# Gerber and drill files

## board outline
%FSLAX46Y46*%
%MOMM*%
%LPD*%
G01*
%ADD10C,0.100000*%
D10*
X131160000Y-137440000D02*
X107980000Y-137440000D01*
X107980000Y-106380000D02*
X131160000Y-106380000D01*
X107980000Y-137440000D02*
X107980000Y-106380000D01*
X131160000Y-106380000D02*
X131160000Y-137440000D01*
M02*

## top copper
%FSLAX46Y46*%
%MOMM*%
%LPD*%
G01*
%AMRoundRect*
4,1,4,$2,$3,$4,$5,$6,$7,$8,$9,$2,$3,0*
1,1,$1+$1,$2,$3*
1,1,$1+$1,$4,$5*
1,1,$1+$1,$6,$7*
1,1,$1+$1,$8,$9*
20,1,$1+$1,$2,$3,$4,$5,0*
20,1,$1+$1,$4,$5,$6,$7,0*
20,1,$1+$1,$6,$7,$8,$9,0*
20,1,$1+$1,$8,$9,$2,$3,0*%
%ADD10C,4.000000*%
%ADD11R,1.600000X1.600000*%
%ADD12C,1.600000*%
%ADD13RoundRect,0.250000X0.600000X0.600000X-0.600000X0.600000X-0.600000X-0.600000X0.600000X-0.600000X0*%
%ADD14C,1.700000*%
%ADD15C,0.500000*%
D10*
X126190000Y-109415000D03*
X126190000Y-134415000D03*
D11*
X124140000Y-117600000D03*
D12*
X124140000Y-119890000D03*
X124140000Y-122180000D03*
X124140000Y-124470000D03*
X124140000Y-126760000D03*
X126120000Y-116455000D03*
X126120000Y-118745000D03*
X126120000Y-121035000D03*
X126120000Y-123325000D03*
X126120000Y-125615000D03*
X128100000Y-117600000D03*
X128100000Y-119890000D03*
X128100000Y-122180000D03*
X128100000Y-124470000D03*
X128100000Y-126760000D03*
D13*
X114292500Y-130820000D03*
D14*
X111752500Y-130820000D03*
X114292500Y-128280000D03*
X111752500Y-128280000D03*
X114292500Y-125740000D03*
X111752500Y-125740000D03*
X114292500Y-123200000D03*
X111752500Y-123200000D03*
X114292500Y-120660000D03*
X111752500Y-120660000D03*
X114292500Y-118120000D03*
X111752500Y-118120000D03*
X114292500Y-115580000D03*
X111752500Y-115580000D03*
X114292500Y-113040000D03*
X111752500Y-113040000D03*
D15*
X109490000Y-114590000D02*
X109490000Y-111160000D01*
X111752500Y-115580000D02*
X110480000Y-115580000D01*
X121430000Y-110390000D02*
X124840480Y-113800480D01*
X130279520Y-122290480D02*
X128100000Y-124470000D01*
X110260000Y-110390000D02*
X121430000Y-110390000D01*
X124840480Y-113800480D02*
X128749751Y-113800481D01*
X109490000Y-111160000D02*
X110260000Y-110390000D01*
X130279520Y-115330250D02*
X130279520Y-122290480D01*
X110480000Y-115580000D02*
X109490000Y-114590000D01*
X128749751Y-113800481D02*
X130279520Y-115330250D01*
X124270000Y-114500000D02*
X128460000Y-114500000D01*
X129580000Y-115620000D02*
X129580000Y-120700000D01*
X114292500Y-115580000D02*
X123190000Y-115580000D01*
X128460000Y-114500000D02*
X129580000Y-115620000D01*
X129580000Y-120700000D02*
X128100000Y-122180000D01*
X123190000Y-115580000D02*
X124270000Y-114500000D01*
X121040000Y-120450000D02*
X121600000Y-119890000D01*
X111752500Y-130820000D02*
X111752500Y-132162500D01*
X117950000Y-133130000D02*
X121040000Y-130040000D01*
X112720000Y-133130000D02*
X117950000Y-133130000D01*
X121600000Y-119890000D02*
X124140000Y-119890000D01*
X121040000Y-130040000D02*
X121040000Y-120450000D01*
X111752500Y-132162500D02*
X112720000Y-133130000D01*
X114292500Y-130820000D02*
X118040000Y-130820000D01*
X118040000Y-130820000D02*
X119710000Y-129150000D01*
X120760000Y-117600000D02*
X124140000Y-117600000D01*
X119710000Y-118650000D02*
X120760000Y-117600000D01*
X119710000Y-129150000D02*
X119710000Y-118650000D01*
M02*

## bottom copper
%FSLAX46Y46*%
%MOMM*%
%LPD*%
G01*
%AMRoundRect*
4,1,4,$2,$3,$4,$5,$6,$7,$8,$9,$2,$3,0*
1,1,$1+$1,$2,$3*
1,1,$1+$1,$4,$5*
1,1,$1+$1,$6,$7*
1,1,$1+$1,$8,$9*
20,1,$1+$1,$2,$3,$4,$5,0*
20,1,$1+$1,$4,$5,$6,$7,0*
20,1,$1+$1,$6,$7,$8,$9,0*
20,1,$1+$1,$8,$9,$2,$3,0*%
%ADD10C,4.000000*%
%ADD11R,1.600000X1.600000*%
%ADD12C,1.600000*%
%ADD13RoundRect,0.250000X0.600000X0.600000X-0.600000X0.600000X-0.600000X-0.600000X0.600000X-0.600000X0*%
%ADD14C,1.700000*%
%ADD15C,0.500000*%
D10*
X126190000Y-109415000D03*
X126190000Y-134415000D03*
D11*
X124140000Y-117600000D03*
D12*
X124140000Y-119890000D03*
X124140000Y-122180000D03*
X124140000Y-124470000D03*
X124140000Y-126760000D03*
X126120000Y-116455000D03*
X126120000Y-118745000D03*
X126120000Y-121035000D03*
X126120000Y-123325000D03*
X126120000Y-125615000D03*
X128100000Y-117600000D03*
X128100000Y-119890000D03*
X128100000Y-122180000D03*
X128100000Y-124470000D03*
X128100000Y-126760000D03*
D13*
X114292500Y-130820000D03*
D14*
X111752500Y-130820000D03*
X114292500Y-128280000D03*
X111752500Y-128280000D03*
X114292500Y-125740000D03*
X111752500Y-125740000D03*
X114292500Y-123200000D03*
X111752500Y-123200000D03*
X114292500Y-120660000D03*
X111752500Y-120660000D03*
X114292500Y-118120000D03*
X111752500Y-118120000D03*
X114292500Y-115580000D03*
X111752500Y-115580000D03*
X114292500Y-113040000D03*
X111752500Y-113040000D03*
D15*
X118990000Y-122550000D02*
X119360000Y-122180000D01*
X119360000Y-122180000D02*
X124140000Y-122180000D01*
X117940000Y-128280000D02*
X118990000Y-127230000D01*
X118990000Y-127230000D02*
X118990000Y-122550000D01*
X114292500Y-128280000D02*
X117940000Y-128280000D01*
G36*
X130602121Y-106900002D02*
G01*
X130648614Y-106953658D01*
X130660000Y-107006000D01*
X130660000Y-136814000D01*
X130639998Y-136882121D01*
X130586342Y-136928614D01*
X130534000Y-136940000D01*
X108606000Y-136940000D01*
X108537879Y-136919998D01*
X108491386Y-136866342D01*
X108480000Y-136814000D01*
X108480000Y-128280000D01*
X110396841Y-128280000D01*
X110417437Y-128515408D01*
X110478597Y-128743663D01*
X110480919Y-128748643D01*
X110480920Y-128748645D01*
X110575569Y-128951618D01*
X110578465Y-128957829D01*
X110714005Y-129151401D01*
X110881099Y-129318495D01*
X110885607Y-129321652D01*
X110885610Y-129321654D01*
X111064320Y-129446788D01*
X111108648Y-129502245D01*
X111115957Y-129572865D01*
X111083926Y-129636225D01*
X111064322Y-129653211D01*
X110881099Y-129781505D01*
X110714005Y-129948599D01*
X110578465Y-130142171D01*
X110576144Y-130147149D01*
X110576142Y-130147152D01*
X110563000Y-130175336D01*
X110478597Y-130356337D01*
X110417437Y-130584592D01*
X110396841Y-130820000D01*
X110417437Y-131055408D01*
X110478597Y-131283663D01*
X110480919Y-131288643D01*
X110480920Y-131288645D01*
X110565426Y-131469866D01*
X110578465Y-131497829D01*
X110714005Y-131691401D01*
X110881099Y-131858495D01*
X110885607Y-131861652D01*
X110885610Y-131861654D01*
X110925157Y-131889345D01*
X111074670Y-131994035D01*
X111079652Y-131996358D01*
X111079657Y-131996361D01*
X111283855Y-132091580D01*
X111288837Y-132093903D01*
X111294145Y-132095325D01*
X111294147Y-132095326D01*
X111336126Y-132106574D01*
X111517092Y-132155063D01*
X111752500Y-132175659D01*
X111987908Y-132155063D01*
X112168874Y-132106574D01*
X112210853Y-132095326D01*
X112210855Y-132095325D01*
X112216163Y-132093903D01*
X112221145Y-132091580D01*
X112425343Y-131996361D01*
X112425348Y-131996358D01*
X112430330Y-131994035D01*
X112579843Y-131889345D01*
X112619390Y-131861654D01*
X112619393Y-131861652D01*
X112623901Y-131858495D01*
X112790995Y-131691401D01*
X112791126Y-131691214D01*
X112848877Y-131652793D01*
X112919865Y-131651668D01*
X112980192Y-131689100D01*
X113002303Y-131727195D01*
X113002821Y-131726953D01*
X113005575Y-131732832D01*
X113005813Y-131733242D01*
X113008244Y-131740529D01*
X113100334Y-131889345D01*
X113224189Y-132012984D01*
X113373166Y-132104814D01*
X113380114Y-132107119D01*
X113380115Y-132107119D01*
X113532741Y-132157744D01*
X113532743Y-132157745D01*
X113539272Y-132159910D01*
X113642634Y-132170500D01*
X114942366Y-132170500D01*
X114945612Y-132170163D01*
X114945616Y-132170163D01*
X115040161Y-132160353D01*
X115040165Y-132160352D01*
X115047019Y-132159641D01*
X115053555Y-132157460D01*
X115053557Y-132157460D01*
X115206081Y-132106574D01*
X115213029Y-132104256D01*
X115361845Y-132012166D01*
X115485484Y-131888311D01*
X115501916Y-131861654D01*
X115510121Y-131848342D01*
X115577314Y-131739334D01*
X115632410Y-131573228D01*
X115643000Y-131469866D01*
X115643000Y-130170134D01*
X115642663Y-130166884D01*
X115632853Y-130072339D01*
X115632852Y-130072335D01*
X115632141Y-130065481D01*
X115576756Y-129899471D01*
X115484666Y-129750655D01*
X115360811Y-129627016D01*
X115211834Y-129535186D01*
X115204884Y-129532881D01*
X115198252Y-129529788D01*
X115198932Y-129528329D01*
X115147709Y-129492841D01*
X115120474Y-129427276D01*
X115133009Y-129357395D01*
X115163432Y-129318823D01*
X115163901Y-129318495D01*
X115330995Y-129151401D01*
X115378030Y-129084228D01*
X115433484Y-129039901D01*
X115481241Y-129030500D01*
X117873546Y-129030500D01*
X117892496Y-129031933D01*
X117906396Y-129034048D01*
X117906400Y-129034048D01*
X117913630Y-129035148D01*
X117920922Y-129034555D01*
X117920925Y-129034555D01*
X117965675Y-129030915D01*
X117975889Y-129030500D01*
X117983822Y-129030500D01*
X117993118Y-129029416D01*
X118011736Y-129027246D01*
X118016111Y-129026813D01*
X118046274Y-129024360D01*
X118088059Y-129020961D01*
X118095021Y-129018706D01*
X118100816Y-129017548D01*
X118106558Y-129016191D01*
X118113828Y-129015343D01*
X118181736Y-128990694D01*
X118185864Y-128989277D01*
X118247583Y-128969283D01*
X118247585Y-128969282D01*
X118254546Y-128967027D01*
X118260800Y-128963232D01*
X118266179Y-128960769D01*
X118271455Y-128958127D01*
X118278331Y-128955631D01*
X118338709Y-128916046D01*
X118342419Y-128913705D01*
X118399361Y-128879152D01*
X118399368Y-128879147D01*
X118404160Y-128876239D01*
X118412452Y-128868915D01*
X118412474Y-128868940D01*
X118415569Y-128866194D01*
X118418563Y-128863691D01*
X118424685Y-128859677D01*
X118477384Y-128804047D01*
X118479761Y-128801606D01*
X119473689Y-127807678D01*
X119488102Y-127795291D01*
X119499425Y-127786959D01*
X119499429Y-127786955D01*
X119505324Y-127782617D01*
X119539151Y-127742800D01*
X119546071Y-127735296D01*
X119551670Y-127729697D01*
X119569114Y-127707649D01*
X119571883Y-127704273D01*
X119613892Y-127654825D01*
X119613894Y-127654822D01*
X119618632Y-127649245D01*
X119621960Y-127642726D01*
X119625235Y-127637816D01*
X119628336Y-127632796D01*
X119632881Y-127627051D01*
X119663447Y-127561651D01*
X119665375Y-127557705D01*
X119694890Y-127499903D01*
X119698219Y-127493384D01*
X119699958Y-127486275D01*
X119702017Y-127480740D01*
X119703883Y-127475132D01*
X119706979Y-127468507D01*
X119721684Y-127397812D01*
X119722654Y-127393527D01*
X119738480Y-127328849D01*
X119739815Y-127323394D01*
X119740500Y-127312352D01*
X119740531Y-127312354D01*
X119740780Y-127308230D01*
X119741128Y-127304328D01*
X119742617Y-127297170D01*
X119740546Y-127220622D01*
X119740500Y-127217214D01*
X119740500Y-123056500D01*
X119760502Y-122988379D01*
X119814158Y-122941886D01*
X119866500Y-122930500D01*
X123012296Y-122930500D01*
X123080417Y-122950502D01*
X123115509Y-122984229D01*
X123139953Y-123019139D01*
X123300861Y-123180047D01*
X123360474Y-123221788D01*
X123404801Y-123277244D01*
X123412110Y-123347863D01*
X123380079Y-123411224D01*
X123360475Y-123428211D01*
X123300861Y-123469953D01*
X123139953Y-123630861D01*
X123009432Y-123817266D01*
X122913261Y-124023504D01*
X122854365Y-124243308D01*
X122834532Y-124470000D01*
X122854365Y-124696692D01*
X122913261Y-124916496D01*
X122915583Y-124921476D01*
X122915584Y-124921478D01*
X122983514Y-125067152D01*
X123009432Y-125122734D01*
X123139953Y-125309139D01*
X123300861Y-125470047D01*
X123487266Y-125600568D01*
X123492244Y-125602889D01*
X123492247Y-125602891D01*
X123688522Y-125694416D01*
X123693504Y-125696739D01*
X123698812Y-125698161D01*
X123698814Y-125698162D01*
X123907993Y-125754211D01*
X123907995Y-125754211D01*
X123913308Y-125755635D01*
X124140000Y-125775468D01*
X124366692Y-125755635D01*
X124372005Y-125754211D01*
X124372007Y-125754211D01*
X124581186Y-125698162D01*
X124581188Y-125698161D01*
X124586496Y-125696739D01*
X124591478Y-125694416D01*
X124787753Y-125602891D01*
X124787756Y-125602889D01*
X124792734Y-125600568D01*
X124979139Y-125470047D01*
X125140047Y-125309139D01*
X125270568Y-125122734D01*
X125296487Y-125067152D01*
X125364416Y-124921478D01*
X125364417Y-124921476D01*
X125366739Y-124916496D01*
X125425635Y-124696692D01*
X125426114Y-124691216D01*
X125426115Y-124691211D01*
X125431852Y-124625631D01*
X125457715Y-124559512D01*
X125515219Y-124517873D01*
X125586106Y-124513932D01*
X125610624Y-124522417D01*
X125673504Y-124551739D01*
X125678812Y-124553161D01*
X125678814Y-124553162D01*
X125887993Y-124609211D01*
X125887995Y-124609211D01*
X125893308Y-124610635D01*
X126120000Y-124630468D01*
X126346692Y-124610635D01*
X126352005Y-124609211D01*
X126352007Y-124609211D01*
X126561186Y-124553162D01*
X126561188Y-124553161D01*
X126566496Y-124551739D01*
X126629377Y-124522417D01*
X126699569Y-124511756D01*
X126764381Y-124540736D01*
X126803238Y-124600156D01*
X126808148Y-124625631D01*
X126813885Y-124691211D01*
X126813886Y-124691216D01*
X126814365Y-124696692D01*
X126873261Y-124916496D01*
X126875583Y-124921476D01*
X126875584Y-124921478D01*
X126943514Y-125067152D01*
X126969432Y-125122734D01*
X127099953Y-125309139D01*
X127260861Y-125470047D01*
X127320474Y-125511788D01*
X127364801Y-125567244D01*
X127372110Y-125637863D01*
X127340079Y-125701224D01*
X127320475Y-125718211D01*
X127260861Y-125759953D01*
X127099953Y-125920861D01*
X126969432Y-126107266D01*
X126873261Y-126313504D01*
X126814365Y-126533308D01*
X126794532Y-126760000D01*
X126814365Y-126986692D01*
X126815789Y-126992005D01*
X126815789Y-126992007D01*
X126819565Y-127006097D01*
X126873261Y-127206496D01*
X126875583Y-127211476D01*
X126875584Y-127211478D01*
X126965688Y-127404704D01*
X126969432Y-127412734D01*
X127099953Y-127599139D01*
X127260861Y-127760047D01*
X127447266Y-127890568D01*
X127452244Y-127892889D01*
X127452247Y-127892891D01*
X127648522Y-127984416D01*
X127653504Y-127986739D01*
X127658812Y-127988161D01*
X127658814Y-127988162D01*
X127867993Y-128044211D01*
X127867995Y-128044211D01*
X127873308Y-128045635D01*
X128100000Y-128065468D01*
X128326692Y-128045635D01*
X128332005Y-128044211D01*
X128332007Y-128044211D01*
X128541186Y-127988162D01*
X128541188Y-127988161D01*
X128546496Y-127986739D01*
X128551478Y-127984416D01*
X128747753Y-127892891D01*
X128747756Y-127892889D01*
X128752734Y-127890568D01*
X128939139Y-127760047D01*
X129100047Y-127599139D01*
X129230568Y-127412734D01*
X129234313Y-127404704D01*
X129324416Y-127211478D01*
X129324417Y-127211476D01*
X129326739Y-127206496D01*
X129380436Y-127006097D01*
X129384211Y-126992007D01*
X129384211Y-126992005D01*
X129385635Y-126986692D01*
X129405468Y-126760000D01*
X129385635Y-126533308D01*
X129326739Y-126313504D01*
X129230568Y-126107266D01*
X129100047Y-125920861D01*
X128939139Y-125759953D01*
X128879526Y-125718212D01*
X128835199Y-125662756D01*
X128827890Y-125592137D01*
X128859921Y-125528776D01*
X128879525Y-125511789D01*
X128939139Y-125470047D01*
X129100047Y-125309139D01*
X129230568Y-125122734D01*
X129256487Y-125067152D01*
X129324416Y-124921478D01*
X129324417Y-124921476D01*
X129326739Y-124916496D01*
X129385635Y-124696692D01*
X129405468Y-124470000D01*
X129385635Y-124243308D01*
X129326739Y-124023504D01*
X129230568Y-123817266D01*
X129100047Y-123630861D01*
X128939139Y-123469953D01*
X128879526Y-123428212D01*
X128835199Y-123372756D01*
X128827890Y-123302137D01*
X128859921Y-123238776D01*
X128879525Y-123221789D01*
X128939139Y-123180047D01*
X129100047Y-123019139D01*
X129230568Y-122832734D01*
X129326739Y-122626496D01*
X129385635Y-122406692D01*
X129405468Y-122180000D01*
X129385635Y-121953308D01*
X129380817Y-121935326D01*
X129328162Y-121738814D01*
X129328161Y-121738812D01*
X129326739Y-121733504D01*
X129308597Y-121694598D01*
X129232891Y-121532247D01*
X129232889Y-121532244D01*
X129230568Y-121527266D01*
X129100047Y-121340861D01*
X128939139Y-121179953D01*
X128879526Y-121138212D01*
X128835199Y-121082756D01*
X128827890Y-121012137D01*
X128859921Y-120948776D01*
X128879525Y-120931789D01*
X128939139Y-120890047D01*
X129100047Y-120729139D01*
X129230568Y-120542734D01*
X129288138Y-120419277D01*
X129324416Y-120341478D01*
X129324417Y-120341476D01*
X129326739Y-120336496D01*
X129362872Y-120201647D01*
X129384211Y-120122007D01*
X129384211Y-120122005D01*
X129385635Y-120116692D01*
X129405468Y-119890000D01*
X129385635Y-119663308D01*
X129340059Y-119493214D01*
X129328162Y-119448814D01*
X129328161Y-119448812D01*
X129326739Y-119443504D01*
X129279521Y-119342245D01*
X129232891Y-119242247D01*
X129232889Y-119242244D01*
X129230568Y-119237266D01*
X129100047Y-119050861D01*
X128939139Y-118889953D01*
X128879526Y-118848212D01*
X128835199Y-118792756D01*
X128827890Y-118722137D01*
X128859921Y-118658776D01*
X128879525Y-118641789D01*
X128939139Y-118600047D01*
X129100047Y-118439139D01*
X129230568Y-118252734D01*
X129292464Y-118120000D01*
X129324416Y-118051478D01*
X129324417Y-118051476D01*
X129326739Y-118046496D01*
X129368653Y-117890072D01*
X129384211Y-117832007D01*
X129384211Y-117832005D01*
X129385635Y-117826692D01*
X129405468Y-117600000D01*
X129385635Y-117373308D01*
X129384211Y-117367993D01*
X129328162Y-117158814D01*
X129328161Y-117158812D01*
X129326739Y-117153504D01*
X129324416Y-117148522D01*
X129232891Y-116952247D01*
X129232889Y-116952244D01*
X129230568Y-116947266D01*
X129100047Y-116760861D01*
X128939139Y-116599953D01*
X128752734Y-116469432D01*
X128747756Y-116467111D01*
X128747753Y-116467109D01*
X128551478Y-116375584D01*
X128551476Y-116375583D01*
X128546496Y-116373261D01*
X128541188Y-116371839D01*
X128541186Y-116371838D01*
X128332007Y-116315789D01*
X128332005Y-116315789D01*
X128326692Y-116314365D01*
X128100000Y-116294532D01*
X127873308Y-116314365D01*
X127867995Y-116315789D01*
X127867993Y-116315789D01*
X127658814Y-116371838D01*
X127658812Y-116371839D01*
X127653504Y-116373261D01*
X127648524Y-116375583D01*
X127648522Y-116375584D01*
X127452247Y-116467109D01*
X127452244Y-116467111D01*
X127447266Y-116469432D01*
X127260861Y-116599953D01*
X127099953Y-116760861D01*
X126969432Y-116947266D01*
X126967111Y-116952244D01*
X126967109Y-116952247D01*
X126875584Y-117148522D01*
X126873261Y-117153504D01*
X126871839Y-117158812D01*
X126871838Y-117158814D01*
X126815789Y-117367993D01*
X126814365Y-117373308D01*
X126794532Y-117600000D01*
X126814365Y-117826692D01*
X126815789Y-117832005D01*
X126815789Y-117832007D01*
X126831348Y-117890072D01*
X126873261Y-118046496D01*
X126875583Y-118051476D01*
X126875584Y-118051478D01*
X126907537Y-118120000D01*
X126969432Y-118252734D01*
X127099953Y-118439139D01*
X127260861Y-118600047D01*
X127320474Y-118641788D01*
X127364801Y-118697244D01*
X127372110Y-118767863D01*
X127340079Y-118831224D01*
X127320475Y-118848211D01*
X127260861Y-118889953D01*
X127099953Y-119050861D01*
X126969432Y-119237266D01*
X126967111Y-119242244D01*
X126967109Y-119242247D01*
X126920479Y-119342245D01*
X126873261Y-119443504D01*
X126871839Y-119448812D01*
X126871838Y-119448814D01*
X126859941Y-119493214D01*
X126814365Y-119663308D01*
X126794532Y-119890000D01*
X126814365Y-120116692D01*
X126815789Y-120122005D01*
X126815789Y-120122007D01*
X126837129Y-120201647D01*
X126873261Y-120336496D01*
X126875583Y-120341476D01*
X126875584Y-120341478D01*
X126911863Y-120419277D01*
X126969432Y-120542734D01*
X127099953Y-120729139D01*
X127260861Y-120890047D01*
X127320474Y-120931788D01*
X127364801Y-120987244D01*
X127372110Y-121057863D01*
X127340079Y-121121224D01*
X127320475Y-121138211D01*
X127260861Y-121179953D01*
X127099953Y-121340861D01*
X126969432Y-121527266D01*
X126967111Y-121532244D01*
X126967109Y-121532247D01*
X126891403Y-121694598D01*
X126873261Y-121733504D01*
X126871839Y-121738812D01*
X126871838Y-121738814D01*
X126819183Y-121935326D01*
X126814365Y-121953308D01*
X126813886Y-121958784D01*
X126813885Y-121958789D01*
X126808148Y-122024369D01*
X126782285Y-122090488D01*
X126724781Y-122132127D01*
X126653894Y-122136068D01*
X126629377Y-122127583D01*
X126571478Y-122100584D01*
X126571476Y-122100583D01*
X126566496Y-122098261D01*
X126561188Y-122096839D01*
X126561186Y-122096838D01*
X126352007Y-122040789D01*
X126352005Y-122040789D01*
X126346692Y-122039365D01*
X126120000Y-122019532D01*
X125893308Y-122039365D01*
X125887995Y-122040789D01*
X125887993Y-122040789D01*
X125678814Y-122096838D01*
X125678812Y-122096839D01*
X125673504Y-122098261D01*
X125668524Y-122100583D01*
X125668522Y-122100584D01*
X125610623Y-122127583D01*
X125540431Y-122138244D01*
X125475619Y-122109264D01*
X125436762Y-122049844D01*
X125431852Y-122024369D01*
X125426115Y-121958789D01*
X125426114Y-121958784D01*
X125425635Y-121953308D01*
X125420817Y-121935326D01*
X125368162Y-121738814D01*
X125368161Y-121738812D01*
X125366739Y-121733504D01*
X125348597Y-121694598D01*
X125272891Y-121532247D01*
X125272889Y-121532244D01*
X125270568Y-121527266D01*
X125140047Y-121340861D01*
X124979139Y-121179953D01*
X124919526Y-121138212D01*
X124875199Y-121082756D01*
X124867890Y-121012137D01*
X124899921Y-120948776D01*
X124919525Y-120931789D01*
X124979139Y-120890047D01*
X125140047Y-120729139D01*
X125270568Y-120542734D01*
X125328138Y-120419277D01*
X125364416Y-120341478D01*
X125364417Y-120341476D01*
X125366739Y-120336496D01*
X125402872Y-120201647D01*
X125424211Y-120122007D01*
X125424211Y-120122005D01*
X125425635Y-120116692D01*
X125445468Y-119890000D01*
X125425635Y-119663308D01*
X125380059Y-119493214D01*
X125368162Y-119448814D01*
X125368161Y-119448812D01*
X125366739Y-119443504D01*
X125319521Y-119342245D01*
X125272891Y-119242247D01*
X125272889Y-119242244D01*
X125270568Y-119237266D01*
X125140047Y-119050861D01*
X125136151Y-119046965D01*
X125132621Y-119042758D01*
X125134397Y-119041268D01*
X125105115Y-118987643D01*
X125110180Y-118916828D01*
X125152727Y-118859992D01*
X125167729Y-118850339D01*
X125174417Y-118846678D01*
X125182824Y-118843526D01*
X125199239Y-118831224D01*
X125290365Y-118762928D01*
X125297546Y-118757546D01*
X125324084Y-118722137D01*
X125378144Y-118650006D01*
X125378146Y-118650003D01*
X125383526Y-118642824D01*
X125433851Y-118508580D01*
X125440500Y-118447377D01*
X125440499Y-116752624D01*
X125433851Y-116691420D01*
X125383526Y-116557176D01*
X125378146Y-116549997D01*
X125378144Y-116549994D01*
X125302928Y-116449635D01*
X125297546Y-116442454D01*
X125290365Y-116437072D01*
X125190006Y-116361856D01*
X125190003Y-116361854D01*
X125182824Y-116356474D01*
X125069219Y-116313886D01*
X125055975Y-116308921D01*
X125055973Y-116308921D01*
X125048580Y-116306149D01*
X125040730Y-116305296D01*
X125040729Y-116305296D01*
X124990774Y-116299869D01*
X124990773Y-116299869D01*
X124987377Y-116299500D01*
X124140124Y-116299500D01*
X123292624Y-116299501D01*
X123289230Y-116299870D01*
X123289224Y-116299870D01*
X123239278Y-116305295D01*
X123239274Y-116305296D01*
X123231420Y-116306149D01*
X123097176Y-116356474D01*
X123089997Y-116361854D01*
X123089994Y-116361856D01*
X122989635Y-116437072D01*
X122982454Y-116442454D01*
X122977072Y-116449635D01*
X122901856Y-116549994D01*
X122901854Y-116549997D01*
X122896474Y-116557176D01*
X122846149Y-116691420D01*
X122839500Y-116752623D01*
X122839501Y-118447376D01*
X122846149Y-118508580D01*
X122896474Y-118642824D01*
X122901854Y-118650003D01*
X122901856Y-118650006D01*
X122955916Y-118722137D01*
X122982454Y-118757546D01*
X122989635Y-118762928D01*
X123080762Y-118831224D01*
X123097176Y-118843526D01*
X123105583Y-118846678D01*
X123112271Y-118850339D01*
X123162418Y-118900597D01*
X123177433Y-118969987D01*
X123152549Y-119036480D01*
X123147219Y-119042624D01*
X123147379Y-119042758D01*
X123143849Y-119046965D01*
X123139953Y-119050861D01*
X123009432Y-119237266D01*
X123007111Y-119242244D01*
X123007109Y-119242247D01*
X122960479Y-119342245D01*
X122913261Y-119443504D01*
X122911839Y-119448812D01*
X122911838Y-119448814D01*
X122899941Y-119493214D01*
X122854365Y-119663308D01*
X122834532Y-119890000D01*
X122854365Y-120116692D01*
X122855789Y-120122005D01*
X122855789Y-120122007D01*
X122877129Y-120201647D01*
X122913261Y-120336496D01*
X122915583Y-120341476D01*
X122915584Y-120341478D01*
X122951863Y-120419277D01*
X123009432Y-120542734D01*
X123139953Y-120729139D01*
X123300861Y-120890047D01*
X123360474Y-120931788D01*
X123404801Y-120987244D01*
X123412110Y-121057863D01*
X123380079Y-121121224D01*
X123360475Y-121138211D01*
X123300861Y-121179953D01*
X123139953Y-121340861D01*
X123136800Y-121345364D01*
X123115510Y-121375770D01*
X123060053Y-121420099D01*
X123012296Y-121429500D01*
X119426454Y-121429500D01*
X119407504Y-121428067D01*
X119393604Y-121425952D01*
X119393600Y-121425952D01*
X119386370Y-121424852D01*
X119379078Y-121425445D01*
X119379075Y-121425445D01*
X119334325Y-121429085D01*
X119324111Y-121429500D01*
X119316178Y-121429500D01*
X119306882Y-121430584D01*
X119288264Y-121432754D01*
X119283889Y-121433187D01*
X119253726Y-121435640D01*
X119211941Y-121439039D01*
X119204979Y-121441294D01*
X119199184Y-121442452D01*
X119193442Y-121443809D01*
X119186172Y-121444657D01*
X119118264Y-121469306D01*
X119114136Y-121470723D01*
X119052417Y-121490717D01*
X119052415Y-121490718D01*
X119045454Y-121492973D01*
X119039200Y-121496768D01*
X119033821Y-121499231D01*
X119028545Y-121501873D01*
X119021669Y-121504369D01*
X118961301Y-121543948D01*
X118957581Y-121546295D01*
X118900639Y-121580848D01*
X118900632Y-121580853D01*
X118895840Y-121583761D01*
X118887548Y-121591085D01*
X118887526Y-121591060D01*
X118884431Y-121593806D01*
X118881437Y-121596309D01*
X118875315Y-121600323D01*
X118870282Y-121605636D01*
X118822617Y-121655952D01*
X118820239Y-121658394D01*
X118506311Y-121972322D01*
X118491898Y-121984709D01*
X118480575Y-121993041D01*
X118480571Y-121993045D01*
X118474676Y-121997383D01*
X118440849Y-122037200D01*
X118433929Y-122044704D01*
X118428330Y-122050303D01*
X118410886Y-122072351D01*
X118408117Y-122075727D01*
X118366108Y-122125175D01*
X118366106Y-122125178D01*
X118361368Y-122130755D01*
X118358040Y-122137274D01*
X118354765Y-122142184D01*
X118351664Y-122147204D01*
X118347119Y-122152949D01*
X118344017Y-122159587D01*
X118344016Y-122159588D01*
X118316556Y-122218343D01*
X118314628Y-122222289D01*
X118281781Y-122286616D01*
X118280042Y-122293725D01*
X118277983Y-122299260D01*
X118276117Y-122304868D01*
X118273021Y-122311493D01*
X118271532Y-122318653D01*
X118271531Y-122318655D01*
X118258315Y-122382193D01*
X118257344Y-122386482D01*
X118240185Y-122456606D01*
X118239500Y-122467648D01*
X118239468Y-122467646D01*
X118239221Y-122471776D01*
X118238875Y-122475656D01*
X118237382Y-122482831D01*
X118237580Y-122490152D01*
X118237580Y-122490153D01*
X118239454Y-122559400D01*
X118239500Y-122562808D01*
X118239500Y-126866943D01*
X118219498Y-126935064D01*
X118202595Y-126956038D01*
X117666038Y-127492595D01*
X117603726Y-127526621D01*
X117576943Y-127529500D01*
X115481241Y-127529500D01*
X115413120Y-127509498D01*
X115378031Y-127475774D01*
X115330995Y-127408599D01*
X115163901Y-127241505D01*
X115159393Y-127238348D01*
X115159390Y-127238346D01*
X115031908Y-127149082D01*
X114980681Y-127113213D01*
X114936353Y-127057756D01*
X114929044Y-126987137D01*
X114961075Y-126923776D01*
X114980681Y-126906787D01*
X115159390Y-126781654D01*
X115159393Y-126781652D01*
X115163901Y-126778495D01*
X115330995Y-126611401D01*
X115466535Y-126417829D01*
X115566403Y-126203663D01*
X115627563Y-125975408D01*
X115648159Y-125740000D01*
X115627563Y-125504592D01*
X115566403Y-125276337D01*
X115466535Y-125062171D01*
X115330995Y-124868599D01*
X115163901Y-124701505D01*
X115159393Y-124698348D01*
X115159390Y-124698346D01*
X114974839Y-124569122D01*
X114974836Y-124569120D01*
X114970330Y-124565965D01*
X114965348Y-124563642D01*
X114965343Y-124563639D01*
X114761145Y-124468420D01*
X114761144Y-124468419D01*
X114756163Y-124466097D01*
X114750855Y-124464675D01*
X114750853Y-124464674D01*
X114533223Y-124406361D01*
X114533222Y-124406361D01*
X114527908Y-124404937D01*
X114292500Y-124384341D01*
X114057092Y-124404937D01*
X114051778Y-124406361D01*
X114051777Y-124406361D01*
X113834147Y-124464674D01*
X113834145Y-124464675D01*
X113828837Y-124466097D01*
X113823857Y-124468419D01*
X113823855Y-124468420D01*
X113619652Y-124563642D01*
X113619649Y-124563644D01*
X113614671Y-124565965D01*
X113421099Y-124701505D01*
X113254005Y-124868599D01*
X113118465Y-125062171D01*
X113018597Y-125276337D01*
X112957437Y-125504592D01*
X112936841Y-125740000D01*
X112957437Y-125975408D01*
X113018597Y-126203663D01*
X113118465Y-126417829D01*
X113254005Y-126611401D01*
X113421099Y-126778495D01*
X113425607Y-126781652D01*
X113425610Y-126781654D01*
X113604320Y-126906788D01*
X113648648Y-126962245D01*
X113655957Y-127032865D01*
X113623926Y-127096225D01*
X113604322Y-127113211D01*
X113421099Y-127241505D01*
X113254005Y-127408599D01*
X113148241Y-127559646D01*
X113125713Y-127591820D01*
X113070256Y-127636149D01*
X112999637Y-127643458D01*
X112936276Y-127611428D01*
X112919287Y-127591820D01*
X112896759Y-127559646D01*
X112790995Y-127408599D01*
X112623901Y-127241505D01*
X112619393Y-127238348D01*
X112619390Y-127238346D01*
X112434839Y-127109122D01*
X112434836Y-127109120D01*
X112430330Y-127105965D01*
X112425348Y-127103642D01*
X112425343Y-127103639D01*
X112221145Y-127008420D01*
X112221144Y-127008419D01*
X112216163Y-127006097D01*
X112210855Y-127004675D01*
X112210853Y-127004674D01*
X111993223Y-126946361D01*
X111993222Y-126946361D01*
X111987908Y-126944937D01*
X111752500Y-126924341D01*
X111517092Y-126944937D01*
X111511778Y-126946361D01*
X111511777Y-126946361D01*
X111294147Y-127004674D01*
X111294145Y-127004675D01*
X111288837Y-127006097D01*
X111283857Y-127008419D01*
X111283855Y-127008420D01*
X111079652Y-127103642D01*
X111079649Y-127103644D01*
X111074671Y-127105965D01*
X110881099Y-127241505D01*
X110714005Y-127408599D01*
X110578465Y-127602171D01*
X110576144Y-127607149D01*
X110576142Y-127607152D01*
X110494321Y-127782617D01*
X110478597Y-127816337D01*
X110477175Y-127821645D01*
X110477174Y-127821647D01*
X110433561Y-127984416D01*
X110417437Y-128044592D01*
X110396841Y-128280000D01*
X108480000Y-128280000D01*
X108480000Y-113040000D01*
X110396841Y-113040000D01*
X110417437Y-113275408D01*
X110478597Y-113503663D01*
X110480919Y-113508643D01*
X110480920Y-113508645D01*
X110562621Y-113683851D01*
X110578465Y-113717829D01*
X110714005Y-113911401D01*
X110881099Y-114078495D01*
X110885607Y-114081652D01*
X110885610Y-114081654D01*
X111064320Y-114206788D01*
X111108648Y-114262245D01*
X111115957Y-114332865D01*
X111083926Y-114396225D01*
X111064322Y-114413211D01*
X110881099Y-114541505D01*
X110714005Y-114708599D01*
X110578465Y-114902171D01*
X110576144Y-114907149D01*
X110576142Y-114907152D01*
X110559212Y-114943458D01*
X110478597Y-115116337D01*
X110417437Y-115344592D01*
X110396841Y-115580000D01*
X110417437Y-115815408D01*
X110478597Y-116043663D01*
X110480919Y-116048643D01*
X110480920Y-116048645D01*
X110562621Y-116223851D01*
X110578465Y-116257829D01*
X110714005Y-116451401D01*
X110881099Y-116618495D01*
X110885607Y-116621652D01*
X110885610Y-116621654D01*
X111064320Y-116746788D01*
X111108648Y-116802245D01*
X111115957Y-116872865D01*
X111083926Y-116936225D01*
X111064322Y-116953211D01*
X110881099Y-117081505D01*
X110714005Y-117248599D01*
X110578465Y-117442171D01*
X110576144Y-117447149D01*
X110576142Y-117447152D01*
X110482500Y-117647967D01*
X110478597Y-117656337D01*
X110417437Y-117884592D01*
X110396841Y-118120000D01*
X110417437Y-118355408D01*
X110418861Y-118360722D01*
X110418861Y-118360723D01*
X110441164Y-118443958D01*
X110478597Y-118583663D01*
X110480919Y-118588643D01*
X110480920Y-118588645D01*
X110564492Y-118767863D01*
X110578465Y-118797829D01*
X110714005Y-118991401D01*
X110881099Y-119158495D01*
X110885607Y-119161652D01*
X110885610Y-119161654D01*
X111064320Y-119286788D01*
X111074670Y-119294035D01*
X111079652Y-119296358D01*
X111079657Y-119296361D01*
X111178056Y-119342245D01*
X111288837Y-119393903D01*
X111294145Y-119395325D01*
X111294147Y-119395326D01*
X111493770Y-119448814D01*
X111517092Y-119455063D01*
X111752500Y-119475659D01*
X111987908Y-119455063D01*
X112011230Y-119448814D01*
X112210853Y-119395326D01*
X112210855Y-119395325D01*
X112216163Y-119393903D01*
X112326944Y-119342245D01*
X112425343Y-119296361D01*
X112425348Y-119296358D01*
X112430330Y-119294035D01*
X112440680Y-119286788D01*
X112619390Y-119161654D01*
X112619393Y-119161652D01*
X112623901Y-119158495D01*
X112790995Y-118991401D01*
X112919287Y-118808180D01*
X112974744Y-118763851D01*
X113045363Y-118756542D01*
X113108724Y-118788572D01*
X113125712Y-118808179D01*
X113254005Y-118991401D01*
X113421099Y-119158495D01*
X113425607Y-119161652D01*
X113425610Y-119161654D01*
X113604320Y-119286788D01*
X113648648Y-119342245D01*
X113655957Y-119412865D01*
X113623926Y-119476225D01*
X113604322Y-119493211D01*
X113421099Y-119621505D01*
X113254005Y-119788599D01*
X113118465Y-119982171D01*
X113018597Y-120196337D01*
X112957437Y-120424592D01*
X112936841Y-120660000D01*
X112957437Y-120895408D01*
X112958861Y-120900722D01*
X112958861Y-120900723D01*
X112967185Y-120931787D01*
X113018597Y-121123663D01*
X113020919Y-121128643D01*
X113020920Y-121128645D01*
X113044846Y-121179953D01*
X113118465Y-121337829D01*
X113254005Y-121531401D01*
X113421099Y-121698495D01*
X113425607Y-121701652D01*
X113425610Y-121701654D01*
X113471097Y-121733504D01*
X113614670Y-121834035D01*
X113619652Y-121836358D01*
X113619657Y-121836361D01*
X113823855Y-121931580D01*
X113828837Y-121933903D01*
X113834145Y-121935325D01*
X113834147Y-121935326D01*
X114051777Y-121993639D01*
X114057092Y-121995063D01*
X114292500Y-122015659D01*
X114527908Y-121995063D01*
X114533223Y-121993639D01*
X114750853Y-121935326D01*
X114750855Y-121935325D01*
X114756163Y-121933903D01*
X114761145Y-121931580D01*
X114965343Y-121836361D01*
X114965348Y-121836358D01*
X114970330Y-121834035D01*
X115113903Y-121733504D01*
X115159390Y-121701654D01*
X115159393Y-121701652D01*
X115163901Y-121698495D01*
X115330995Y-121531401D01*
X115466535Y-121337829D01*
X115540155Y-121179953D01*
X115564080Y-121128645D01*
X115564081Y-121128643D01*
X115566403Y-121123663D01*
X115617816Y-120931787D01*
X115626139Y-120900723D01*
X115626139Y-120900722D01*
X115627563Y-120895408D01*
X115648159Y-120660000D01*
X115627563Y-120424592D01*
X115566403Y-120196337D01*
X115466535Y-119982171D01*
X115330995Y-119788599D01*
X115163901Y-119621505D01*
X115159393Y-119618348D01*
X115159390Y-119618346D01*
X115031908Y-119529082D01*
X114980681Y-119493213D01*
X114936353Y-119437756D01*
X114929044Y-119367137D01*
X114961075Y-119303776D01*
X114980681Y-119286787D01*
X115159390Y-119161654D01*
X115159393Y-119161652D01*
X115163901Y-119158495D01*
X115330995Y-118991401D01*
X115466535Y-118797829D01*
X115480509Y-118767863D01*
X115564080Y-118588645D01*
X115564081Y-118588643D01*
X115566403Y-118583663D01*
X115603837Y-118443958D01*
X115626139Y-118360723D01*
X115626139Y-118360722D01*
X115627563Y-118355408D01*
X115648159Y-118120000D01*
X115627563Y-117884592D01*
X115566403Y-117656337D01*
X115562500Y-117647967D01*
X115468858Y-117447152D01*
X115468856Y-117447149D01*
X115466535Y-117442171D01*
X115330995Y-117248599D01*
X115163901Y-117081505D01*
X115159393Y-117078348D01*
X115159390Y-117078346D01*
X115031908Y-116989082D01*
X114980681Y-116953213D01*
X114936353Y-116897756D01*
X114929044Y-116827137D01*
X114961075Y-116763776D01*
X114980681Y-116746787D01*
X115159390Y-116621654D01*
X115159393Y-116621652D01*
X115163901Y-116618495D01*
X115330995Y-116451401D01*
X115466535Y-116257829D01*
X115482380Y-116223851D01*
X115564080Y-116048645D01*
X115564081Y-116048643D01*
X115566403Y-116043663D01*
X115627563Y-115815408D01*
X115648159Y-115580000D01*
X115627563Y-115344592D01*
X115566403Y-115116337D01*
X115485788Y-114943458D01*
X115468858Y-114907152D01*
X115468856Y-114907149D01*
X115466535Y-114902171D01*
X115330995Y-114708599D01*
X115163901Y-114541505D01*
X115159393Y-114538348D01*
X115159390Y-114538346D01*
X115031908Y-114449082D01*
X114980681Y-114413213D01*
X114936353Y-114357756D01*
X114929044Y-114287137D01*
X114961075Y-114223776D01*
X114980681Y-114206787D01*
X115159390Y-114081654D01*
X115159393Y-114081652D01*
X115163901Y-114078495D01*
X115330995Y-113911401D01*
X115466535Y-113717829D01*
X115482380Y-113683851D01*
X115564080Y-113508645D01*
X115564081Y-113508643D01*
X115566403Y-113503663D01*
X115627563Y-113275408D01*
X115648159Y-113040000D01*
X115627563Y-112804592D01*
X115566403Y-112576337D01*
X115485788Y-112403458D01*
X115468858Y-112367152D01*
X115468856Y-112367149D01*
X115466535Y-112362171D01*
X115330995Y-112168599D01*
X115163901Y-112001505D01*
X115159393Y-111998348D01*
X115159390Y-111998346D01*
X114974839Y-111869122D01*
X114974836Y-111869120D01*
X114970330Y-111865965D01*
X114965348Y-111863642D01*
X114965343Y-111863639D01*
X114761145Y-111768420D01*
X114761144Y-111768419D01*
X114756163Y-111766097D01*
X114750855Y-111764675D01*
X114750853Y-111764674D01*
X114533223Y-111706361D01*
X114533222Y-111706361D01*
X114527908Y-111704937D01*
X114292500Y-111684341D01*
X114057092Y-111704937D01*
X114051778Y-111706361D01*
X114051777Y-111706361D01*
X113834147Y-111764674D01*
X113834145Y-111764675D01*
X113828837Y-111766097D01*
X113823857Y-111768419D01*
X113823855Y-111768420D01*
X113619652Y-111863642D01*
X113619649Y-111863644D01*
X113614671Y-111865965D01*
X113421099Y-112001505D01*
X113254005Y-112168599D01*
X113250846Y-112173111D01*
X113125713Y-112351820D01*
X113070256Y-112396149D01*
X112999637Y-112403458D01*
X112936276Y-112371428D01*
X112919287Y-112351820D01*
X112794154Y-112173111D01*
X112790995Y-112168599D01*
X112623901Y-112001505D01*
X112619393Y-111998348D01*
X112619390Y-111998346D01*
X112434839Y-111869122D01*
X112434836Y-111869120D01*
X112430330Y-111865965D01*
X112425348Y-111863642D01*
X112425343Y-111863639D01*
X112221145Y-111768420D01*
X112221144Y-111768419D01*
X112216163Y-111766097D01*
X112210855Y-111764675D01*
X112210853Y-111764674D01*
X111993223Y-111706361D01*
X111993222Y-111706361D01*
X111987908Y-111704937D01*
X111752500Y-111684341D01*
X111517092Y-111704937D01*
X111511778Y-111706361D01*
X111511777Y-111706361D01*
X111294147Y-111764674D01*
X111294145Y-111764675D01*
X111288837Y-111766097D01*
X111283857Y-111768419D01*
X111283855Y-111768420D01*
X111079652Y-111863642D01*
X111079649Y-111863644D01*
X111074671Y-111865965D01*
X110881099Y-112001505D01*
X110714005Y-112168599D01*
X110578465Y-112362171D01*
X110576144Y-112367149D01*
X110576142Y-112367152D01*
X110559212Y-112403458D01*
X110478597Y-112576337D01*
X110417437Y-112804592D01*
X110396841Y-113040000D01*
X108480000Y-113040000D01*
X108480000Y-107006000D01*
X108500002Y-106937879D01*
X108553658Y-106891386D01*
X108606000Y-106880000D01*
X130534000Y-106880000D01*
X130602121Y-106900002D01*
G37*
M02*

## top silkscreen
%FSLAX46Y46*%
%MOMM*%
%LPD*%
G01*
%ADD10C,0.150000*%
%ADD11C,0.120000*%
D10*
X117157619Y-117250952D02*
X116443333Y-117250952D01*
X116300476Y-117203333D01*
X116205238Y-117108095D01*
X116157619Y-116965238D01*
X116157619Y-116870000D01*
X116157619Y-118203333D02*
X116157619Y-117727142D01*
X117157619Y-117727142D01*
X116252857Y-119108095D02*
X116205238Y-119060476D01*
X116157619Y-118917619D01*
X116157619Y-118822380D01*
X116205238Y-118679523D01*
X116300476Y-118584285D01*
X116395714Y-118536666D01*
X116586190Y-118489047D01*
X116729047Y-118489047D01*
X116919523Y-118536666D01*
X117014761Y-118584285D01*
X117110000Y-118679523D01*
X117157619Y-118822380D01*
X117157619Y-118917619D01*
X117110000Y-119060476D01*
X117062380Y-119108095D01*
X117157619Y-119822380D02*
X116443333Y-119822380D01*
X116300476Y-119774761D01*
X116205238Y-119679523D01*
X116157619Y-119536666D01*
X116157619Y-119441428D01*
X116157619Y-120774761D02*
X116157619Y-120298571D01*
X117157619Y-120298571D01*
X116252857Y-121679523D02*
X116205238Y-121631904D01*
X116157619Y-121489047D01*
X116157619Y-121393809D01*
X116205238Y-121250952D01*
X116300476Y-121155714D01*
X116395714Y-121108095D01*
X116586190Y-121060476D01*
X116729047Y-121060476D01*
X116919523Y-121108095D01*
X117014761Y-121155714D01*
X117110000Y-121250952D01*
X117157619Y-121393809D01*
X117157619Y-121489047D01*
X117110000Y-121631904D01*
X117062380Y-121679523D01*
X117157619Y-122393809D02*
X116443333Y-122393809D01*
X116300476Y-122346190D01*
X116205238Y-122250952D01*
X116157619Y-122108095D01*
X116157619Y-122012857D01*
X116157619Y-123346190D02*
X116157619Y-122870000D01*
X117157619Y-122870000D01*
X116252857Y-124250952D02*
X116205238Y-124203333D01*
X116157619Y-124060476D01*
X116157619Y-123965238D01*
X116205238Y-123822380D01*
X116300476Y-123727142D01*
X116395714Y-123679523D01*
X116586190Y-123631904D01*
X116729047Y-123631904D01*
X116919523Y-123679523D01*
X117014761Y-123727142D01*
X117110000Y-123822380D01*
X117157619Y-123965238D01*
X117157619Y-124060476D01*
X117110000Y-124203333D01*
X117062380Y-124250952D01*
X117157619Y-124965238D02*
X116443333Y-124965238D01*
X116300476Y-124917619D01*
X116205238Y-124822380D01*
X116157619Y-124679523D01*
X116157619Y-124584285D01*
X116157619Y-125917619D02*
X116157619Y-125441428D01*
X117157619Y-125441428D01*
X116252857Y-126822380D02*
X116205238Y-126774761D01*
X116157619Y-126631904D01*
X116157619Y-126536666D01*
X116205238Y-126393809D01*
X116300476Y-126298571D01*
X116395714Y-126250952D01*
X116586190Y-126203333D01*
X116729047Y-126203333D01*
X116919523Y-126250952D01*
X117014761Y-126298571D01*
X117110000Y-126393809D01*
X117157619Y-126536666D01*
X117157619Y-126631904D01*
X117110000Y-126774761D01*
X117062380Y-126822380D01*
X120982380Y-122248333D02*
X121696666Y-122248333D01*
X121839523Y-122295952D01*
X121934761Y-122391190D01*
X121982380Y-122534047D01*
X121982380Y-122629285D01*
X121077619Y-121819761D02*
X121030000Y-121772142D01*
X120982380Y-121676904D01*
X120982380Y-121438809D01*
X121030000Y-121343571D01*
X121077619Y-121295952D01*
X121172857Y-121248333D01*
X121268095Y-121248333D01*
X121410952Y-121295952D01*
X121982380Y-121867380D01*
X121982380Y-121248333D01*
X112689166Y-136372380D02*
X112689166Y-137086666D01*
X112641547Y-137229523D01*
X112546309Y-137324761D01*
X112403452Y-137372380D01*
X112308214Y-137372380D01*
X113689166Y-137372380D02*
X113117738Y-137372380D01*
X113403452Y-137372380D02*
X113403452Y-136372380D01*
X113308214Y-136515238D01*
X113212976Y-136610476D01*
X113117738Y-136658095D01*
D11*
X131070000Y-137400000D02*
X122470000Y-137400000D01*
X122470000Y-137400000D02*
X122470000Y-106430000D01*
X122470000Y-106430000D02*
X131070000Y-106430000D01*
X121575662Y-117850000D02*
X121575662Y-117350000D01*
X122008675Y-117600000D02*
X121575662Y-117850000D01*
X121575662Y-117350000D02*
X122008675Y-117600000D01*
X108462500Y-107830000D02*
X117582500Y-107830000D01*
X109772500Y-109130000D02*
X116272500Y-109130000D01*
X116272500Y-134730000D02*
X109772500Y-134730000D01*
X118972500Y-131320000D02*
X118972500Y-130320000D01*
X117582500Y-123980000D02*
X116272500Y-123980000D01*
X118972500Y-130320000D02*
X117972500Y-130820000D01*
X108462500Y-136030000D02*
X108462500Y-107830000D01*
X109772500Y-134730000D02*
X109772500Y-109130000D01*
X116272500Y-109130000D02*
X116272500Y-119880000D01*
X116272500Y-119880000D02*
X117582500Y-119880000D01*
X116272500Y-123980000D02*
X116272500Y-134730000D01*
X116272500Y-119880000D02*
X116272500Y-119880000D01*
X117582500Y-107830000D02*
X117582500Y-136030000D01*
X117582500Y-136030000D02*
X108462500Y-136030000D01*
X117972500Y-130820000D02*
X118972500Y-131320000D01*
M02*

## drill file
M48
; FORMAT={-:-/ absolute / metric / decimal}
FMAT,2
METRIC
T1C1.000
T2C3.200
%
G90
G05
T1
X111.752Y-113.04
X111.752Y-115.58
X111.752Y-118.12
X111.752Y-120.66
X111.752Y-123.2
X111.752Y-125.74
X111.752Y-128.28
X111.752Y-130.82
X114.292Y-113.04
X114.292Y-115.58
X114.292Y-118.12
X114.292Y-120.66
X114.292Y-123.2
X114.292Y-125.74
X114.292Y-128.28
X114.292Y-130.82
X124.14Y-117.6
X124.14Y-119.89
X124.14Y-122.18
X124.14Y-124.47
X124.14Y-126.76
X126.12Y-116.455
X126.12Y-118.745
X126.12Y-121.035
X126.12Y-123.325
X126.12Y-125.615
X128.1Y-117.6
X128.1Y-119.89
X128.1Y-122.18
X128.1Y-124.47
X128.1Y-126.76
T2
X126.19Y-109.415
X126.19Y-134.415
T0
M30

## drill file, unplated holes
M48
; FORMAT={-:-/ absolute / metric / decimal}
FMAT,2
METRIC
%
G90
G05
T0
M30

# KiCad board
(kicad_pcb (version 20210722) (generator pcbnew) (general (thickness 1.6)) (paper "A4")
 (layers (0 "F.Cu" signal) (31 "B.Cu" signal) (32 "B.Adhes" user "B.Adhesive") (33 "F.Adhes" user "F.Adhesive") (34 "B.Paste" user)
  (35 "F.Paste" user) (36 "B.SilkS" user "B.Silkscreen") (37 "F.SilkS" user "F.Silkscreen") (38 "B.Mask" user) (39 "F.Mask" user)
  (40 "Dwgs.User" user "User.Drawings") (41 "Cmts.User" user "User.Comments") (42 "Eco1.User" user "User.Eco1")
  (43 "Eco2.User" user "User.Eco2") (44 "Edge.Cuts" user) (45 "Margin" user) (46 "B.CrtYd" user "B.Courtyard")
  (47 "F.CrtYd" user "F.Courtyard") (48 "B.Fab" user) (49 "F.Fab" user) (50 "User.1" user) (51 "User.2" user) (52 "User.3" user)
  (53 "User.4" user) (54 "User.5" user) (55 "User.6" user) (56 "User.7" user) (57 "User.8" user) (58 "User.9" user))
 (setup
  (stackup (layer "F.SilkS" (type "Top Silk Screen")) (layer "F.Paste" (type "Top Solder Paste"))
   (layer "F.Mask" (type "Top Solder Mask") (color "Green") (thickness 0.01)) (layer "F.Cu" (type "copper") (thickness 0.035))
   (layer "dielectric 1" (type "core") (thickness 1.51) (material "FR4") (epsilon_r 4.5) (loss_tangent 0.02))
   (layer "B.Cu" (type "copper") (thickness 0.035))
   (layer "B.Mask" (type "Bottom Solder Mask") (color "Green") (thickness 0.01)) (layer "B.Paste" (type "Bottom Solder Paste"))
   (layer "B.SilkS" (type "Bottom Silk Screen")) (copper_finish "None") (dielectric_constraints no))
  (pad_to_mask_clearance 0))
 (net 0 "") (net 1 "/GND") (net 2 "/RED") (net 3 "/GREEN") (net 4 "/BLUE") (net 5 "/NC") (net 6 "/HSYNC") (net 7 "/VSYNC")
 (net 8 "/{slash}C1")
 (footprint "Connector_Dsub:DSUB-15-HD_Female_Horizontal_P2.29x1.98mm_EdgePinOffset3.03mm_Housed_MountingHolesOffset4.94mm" (layer "F.Cu")
  (at 124.14 117.6 90)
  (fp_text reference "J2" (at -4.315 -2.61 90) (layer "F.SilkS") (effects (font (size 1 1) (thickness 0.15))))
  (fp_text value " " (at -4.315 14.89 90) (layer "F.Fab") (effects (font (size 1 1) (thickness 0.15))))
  (fp_line (start -19.8 6.93) (end -19.8 -1.67) (layer "F.SilkS") (width 0.12))
  (fp_line (start -19.8 -1.67) (end 11.17 -1.67) (layer "F.SilkS") (width 0.12))
  (fp_line (start 11.17 -1.67) (end 11.17 6.93) (layer "F.SilkS") (width 0.12))
  (fp_line (start -0.25 -2.564338) (end 0.25 -2.564338) (layer "F.SilkS") (width 0.12))
  (fp_line (start 0 -2.131325) (end -0.25 -2.564338) (layer "F.SilkS") (width 0.12))
  (fp_line (start 0.25 -2.564338) (end 0 -2.131325) (layer "F.SilkS") (width 0.12))
  (pad "0" thru_hole circle locked (at 8.185 2.05 90) (size 4 4) (drill 3.2) (layers *.Cu *.Mask) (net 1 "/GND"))
  (pad "0" thru_hole circle locked (at -16.815 2.05 90) (size 4 4) (drill 3.2) (layers *.Cu *.Mask) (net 1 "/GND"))
  (pad "1" thru_hole rect locked (at 0 0 90) (size 1.6 1.6) (drill 1) (layers *.Cu *.Mask) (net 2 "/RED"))
  (pad "2" thru_hole circle locked (at -2.29 0 90) (size 1.6 1.6) (drill 1) (layers *.Cu *.Mask) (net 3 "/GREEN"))
  (pad "3" thru_hole circle locked (at -4.58 0 90) (size 1.6 1.6) (drill 1) (layers *.Cu *.Mask) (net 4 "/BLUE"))
  (pad "4" thru_hole circle locked (at -6.87 0 90) (size 1.6 1.6) (drill 1) (layers *.Cu *.Mask) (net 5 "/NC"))
  (pad "5" thru_hole circle locked (at -9.16 0 90) (size 1.6 1.6) (drill 1) (layers *.Cu *.Mask) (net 1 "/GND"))
  (pad "6" thru_hole circle locked (at 1.145 1.98 90) (size 1.6 1.6) (drill 1) (layers *.Cu *.Mask) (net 1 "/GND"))
  (pad "7" thru_hole circle locked (at -1.145 1.98 90) (size 1.6 1.6) (drill 1) (layers *.Cu *.Mask) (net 1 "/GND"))
  (pad "8" thru_hole circle locked (at -3.435 1.98 90) (size 1.6 1.6) (drill 1) (layers *.Cu *.Mask) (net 1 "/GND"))
  (pad "9" thru_hole circle locked (at -5.725 1.98 90) (size 1.6 1.6) (drill 1) (layers *.Cu *.Mask) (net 5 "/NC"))
  (pad "10" thru_hole circle locked (at -8.015 1.98 90) (size 1.6 1.6) (drill 1) (layers *.Cu *.Mask) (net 1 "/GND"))
  (pad "11" thru_hole circle locked (at 0 3.96 90) (size 1.6 1.6) (drill 1) (layers *.Cu *.Mask) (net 5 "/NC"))
  (pad "12" thru_hole circle locked (at -2.29 3.96 90) (size 1.6 1.6) (drill 1) (layers *.Cu *.Mask) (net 5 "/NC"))
  (pad "13" thru_hole circle locked (at -4.58 3.96 90) (size 1.6 1.6) (drill 1) (layers *.Cu *.Mask) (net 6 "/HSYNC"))
  (pad "14" thru_hole circle locked (at -6.87 3.96 90) (size 1.6 1.6) (drill 1) (layers *.Cu *.Mask) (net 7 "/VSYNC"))
  (pad "15" thru_hole circle locked (at -9.16 3.96 90) (size 1.6 1.6) (drill 1) (layers *.Cu *.Mask) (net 5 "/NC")))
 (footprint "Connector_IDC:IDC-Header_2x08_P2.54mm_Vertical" (layer "F.Cu") (at 114.2925 130.82 180)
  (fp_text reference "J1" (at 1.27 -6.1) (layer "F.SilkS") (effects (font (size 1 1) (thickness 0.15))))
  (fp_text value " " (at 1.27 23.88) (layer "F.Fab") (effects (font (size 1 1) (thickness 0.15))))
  (fp_line (start 5.83 22.99) (end -3.29 22.99) (layer "F.SilkS") (width 0.12))
  (fp_line (start 4.52 21.69) (end -1.98 21.69) (layer "F.SilkS") (width 0.12))
  (fp_line (start -1.98 -3.91) (end 4.52 -3.91) (layer "F.SilkS") (width 0.12))
  (fp_line (start -4.68 -0.5) (end -4.68 0.5) (layer "F.SilkS") (width 0.12))
  (fp_line (start -3.29 6.84) (end -1.98 6.84) (layer "F.SilkS") (width 0.12))
  (fp_line (start -4.68 0.5) (end -3.68 0) (layer "F.SilkS") (width 0.12))
  (fp_line (start 5.83 -5.21) (end 5.83 22.99) (layer "F.SilkS") (width 0.12))
  (fp_line (start 4.52 -3.91) (end 4.52 21.69) (layer "F.SilkS") (width 0.12))
  (fp_line (start -1.98 21.69) (end -1.98 10.94) (layer "F.SilkS") (width 0.12))
  (fp_line (start -1.98 10.94) (end -3.29 10.94) (layer "F.SilkS") (width 0.12))
  (fp_line (start -1.98 6.84) (end -1.98 -3.91) (layer "F.SilkS") (width 0.12))
  (fp_line (start -1.98 10.94) (end -1.98 10.94) (layer "F.SilkS") (width 0.12))
  (fp_line (start -3.29 22.99) (end -3.29 -5.21) (layer "F.SilkS") (width 0.12))
  (fp_line (start -3.29 -5.21) (end 5.83 -5.21) (layer "F.SilkS") (width 0.12))
  (fp_line (start -3.68 0) (end -4.68 -0.5) (layer "F.SilkS") (width 0.12))
  (pad "1" thru_hole roundrect locked (at 0 0 180) (size 1.7 1.7) (drill 1) (layers *.Cu *.Mask) (roundrect_rratio 0.1470588235)
   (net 2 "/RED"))
  (pad "2" thru_hole circle locked (at 2.54 0 180) (size 1.7 1.7) (drill 1) (layers *.Cu *.Mask) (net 3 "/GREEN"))
  (pad "3" thru_hole circle locked (at 0 2.54 180) (size 1.7 1.7) (drill 1) (layers *.Cu *.Mask) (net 4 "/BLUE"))
  (pad "4" thru_hole circle locked (at 2.54 2.54 180) (size 1.7 1.7) (drill 1) (layers *.Cu *.Mask) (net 5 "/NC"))
  (pad "5" thru_hole circle locked (at 0 5.08 180) (size 1.7 1.7) (drill 1) (layers *.Cu *.Mask) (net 5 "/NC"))
  (pad "6" thru_hole circle locked (at 2.54 5.08 180) (size 1.7 1.7) (drill 1) (layers *.Cu *.Mask) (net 1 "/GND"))
  (pad "7" thru_hole circle locked (at 0 7.62 180) (size 1.7 1.7) (drill 1) (layers *.Cu *.Mask) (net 1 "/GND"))
  (pad "8" thru_hole circle locked (at 2.54 7.62 180) (size 1.7 1.7) (drill 1) (layers *.Cu *.Mask) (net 1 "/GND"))
  (pad "9" thru_hole circle locked (at 0 10.16 180) (size 1.7 1.7) (drill 1) (layers *.Cu *.Mask) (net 5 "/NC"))
  (pad "10" thru_hole circle locked (at 2.54 10.16 180) (size 1.7 1.7) (drill 1) (layers *.Cu *.Mask) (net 1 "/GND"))
  (pad "11" thru_hole circle locked (at 0 12.7 180) (size 1.7 1.7) (drill 1) (layers *.Cu *.Mask) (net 5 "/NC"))
  (pad "12" thru_hole circle locked (at 2.54 12.7 180) (size 1.7 1.7) (drill 1) (layers *.Cu *.Mask) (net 5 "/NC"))
  (pad "13" thru_hole circle locked (at 0 15.24 180) (size 1.7 1.7) (drill 1) (layers *.Cu *.Mask) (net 6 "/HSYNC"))
  (pad "14" thru_hole circle locked (at 2.54 15.24 180) (size 1.7 1.7) (drill 1) (layers *.Cu *.Mask) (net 7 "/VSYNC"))
  (pad "15" thru_hole circle locked (at 0 17.78 180) (size 1.7 1.7) (drill 1) (layers *.Cu *.Mask) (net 5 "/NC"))
  (pad "16" thru_hole circle locked (at 2.54 17.78 180) (size 1.7 1.7) (drill 1) (layers *.Cu *.Mask) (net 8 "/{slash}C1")))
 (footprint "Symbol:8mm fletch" (layer "B.Cu") (at 119.66 110.81 180)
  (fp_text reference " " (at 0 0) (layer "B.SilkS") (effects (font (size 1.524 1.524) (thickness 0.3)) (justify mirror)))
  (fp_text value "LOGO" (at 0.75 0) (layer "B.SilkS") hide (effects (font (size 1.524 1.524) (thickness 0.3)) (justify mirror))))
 (gr_line (start 131.16 137.44) (end 107.98 137.44) (layer "Edge.Cuts") (width 0.1))
 (gr_line (start 107.98 106.38) (end 131.16 106.38) (layer "Edge.Cuts") (width 0.1))
 (gr_line (start 107.98 137.44) (end 107.98 106.38) (layer "Edge.Cuts") (width 0.1))
 (gr_line (start 131.16 106.38) (end 131.16 137.44) (layer "Edge.Cuts") (width 0.1))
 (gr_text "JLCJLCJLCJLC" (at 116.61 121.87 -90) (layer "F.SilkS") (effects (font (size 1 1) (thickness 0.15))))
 (segment (start 109.49 114.59) (end 109.49 111.16) (width 0.5) (layer "F.Cu") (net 7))
 (segment (start 111.7525 115.58) (end 110.48 115.58) (width 0.5) (layer "F.Cu") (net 7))
 (segment (start 121.43 110.39) (end 124.84048 113.80048) (width 0.5) (layer "F.Cu") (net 7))
 (segment (start 130.27952 122.29048) (end 128.1 124.47) (width 0.5) (layer "F.Cu") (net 7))
 (segment (start 110.26 110.39) (end 121.43 110.39) (width 0.5) (layer "F.Cu") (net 7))
 (segment (start 124.84048 113.80048) (end 128.749751 113.800481) (width 0.5) (layer "F.Cu") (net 7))
 (segment (start 109.49 111.16) (end 110.26 110.39) (width 0.5) (layer "F.Cu") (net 7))
 (segment (start 130.27952 115.33025) (end 130.27952 122.29048) (width 0.5) (layer "F.Cu") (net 7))
 (segment (start 110.48 115.58) (end 109.49 114.59) (width 0.5) (layer "F.Cu") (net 7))
 (segment (start 128.749751 113.800481) (end 130.27952 115.33025) (width 0.5) (layer "F.Cu") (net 7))
 (segment (start 124.27 114.5) (end 128.46 114.5) (width 0.5) (layer "F.Cu") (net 6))
 (segment (start 129.58 115.62) (end 129.58 120.7) (width 0.5) (layer "F.Cu") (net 6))
 (segment (start 114.2925 115.58) (end 123.19 115.58) (width 0.5) (layer "F.Cu") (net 6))
 (segment (start 128.46 114.5) (end 129.58 115.62) (width 0.5) (layer "F.Cu") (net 6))
 (segment (start 129.58 120.7) (end 128.1 122.18) (width 0.5) (layer "F.Cu") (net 6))
 (segment (start 123.19 115.58) (end 124.27 114.5) (width 0.5) (layer "F.Cu") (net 6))
 (segment (start 118.99 122.55) (end 119.36 122.18) (width 0.5) (layer "B.Cu") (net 4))
 (segment (start 119.36 122.18) (end 124.14 122.18) (width 0.5) (layer "B.Cu") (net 4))
 (segment (start 117.94 128.28) (end 118.99 127.23) (width 0.5) (layer "B.Cu") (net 4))
 (segment (start 118.99 127.23) (end 118.99 122.55) (width 0.5) (layer "B.Cu") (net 4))
 (segment (start 114.2925 128.28) (end 117.94 128.28) (width 0.5) (layer "B.Cu") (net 4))
 (segment (start 121.04 120.45) (end 121.6 119.89) (width 0.5) (layer "F.Cu") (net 3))
 (segment (start 111.7525 130.82) (end 111.7525 132.1625) (width 0.5) (layer "F.Cu") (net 3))
 (segment (start 117.95 133.13) (end 121.04 130.04) (width 0.5) (layer "F.Cu") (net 3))
 (segment (start 112.72 133.13) (end 117.95 133.13) (width 0.5) (layer "F.Cu") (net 3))
 (segment (start 121.6 119.89) (end 124.14 119.89) (width 0.5) (layer "F.Cu") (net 3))
 (segment (start 121.04 130.04) (end 121.04 120.45) (width 0.5) (layer "F.Cu") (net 3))
 (segment (start 111.7525 132.1625) (end 112.72 133.13) (width 0.5) (layer "F.Cu") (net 3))
 (segment (start 114.2925 130.82) (end 118.04 130.82) (width 0.5) (layer "F.Cu") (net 2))
 (segment (start 118.04 130.82) (end 119.71 129.15) (width 0.5) (layer "F.Cu") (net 2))
 (segment (start 120.76 117.6) (end 124.14 117.6) (width 0.5) (layer "F.Cu") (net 2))
 (segment (start 119.71 118.65) (end 120.76 117.6) (width 0.5) (layer "F.Cu") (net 2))
 (segment (start 119.71 129.15) (end 119.71 118.65) (width 0.5) (layer "F.Cu") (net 2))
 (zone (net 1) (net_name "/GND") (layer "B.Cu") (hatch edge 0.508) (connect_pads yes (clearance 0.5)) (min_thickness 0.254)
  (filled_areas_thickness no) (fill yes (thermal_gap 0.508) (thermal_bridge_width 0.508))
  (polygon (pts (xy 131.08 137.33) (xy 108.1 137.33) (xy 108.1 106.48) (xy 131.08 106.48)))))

